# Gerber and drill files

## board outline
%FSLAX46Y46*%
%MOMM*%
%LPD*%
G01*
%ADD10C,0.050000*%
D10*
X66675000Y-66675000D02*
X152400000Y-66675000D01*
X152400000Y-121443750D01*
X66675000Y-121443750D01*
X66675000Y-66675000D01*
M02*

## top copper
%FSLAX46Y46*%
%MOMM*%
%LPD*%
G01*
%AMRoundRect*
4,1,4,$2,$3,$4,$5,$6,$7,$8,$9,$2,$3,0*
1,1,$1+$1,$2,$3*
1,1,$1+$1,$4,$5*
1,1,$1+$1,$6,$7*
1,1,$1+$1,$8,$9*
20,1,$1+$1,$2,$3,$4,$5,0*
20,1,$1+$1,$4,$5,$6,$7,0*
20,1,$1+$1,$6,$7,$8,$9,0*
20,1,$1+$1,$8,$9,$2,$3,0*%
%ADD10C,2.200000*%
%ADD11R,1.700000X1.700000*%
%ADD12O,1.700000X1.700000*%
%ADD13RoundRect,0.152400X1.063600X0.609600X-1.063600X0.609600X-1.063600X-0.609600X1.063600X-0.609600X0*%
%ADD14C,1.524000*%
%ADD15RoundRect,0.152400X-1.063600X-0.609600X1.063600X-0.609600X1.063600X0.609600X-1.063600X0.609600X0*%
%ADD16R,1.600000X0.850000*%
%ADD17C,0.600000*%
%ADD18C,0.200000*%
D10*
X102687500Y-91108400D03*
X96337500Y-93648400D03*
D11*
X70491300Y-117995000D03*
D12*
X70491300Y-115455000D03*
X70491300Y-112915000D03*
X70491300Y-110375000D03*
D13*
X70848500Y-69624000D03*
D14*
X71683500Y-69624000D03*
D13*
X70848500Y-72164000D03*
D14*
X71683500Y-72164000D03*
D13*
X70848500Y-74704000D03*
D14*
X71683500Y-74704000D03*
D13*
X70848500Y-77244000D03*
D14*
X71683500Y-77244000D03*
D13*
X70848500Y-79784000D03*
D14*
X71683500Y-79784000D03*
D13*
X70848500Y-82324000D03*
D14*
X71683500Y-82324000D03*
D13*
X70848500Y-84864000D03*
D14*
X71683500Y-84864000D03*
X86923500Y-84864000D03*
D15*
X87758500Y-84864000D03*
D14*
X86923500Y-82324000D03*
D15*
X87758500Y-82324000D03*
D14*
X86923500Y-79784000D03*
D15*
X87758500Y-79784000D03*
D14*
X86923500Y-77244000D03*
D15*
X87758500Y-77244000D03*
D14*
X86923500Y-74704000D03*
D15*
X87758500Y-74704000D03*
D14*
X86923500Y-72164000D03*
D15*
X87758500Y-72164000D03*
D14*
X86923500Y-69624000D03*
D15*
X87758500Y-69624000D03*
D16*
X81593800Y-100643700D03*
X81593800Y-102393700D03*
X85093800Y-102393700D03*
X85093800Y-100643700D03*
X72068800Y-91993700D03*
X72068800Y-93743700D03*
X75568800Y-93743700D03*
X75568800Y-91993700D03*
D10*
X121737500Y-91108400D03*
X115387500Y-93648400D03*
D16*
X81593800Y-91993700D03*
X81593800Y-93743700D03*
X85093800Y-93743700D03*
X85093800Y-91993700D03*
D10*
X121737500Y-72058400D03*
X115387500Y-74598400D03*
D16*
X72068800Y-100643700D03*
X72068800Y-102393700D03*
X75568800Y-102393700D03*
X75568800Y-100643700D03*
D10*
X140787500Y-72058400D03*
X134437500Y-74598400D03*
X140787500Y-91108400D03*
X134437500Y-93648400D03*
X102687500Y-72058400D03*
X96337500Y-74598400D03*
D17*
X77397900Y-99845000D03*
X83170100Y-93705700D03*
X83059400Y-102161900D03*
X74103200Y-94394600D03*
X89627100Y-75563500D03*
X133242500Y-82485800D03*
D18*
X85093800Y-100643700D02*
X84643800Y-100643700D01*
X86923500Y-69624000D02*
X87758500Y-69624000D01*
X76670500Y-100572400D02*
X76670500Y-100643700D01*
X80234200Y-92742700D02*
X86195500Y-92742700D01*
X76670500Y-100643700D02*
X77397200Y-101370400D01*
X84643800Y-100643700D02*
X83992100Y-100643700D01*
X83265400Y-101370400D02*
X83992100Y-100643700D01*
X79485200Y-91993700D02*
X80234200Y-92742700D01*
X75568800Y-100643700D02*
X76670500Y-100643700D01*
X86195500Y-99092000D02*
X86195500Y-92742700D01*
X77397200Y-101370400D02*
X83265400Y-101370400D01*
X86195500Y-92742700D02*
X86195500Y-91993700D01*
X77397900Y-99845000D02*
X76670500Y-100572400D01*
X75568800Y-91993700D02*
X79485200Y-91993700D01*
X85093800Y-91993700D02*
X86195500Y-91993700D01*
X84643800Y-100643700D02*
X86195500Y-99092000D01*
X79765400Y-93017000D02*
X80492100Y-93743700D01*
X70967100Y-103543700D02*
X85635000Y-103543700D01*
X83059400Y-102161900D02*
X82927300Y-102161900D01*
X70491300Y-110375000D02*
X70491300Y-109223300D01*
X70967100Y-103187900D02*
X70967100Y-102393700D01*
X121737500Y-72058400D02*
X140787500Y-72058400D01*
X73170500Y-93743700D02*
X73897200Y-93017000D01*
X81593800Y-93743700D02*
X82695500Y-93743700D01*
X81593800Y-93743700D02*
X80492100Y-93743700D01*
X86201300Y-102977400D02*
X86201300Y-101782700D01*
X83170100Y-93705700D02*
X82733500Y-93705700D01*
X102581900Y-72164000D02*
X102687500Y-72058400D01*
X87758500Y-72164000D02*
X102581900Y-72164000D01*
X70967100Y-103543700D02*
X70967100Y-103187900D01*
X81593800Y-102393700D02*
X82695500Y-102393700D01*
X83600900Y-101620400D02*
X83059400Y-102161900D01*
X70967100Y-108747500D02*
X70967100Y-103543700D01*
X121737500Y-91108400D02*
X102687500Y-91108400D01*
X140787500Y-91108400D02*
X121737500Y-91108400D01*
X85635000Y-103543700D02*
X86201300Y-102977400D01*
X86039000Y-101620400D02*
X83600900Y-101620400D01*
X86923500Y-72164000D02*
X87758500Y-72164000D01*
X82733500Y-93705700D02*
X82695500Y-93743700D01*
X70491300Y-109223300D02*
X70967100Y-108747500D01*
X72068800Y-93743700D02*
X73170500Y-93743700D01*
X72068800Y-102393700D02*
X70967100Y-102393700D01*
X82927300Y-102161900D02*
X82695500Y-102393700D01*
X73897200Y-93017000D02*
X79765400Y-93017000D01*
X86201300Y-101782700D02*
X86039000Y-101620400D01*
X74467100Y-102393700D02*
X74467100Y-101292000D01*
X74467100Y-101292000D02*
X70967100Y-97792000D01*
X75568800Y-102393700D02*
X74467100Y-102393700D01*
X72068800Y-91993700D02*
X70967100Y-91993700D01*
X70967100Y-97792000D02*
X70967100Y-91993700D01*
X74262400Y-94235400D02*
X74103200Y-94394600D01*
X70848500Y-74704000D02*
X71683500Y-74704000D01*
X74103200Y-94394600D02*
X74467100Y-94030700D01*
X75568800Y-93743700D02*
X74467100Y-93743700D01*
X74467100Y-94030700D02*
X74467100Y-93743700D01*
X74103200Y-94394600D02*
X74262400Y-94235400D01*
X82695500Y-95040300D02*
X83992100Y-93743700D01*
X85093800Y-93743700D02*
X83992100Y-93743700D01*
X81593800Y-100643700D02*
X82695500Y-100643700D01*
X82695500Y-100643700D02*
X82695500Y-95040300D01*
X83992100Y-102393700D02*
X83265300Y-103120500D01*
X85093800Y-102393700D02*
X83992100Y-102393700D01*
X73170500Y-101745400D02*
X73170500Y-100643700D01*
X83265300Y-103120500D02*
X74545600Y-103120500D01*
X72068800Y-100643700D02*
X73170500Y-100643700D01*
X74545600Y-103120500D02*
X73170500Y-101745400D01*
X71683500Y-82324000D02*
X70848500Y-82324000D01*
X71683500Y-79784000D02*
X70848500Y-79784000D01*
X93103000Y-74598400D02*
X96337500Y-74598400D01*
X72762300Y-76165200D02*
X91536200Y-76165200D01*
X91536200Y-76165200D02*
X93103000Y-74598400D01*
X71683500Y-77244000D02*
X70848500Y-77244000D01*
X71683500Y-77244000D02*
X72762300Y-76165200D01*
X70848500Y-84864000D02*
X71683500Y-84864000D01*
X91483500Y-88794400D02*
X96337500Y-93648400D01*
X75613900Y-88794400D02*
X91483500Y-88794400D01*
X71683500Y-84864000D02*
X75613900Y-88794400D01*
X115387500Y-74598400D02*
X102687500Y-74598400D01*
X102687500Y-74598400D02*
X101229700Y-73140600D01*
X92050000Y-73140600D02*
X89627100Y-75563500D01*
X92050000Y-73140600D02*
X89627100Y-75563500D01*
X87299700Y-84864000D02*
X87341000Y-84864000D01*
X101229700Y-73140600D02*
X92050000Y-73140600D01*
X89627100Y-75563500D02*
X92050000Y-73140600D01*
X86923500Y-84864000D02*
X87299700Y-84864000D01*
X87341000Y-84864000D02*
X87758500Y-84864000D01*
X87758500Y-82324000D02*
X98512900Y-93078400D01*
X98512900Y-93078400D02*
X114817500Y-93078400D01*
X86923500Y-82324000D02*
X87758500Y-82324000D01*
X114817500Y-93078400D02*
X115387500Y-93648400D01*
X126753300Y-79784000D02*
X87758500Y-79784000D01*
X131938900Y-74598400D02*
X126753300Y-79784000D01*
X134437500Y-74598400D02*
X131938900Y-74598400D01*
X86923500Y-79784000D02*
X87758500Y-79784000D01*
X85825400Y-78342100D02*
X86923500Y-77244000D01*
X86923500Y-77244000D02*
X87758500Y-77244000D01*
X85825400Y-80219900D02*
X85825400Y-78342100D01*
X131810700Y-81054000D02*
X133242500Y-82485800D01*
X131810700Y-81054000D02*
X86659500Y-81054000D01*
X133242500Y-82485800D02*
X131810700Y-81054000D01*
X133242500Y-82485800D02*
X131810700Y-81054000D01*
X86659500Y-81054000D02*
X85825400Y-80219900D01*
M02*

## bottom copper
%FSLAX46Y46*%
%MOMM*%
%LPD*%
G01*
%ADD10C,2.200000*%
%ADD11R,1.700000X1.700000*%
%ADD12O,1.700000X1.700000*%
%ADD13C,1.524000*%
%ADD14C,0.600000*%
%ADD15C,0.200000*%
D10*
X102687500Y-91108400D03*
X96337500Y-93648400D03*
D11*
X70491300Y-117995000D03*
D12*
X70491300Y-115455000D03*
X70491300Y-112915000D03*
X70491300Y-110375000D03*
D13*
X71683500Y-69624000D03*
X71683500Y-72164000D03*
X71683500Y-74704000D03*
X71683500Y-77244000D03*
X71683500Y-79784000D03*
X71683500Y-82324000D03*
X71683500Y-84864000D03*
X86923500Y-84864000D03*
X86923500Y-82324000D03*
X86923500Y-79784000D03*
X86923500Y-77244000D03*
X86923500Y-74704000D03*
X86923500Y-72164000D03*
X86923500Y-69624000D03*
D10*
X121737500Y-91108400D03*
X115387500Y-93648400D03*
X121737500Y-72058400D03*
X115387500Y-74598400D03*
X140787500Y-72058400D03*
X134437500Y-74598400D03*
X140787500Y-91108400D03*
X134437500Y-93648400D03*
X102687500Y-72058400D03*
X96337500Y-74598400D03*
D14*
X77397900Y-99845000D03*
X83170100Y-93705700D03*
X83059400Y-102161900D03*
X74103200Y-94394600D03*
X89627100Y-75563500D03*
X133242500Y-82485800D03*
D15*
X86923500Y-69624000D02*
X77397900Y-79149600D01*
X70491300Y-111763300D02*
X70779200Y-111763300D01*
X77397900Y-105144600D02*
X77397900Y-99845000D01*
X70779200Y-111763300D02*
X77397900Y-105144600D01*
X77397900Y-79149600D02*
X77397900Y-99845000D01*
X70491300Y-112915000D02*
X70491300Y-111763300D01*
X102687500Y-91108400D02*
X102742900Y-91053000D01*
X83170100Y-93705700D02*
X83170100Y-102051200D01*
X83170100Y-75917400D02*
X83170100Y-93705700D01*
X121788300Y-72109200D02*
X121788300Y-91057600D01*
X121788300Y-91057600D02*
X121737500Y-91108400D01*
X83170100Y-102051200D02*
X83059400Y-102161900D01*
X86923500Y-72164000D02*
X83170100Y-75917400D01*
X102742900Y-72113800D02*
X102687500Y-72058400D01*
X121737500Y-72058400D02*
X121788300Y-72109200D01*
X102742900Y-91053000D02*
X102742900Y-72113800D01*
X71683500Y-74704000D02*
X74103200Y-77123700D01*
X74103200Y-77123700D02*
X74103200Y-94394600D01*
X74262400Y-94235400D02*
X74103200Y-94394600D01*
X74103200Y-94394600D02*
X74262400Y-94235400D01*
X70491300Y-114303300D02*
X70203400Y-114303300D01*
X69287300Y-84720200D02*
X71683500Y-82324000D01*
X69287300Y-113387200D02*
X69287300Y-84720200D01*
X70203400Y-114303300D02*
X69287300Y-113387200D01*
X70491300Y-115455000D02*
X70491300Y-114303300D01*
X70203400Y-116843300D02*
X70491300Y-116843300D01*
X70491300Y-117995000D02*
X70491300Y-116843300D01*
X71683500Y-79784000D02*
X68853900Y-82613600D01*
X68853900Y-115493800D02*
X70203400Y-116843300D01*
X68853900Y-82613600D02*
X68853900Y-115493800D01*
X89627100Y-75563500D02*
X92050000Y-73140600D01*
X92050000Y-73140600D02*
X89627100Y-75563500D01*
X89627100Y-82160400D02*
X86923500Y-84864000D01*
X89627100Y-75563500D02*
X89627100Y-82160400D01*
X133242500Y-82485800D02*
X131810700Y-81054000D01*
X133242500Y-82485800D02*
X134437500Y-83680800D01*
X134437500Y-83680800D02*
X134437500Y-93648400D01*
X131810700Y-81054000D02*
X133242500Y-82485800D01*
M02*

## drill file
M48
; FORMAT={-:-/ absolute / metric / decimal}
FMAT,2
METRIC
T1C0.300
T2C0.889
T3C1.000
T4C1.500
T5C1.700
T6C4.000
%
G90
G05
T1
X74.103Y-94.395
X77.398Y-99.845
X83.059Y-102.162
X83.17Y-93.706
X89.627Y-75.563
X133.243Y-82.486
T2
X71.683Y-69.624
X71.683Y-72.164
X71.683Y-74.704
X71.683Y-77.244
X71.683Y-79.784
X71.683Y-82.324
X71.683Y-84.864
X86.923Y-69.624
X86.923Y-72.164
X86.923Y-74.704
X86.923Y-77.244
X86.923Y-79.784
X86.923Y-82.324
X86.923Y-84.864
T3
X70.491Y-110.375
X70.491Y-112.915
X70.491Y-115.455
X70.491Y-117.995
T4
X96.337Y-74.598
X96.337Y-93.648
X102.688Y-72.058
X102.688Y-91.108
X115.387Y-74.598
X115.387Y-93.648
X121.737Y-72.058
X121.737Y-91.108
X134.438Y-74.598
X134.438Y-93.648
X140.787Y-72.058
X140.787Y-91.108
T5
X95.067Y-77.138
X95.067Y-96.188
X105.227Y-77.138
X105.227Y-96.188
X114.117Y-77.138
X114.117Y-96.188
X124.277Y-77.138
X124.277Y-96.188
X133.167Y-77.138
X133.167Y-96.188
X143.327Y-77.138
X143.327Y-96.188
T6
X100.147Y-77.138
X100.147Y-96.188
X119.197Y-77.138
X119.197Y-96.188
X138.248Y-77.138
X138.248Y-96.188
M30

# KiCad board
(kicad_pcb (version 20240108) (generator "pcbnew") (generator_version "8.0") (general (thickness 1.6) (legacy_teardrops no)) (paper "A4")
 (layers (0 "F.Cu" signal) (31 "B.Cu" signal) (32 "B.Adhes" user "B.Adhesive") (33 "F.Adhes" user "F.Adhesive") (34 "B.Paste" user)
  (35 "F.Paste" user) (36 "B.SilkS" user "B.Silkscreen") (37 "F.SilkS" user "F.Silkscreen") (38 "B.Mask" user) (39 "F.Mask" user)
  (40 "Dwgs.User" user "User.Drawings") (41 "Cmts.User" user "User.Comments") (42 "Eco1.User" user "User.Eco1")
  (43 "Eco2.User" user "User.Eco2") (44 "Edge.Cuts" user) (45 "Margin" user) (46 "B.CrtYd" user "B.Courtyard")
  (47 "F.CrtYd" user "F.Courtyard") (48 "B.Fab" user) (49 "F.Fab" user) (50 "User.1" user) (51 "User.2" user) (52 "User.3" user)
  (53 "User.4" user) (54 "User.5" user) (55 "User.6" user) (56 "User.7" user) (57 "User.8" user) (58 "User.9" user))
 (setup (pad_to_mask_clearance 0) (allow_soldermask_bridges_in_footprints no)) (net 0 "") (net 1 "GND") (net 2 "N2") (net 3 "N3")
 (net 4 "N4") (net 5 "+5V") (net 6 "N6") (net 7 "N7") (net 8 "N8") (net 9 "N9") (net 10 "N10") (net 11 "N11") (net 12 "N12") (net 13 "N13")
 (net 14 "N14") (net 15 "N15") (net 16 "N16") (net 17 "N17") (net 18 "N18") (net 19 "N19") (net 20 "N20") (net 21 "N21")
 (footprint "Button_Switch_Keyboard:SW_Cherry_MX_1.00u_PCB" (layer "F.Cu") (at 102.6875 91.1084)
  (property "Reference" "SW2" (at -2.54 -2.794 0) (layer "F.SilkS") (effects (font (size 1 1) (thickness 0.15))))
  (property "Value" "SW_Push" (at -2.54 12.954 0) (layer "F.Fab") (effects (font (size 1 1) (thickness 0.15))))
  (pad "" np_thru_hole circle (at -7.62 5.08) (size 1.7 1.7) (drill 1.7) (layers "*.Cu" "*.Mask"))
  (pad "" np_thru_hole circle (at -2.54 5.08) (size 4 4) (drill 4) (layers "*.Cu" "*.Mask"))
  (pad "" np_thru_hole circle (at 2.54 5.08) (size 1.7 1.7) (drill 1.7) (layers "*.Cu" "*.Mask"))
  (pad "1" thru_hole circle (at 0 0) (size 2.2 2.2) (drill 1.5) (layers "*.Cu" "*.Mask") (remove_unused_layers no) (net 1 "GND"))
  (pad "2" thru_hole circle (at -6.35 2.54) (size 2.2 2.2) (drill 1.5) (layers "*.Cu" "*.Mask") (remove_unused_layers no) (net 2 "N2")))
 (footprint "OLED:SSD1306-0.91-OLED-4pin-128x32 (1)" (layer "F.Cu") (at 106.9913 120.185 180)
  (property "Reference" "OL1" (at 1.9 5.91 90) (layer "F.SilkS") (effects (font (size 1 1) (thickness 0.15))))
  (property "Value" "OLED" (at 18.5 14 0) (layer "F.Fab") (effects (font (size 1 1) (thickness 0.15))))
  (pad "1" thru_hole rect (at 36.5 2.19 180) (size 1.7 1.7) (drill 1) (layers "*.Cu" "*.Mask") (remove_unused_layers no) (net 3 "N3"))
  (pad "2" thru_hole oval (at 36.5 4.73 180) (size 1.7 1.7) (drill 1) (layers "*.Cu" "*.Mask") (remove_unused_layers no) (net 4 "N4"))
  (pad "3" thru_hole oval (at 36.5 7.27 180) (size 1.7 1.7) (drill 1) (layers "*.Cu" "*.Mask") (remove_unused_layers no) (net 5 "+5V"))
  (pad "4" thru_hole oval (at 36.5 9.81 180) (size 1.7 1.7) (drill 1) (layers "*.Cu" "*.Mask") (remove_unused_layers no) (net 1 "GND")))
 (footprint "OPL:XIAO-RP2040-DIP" (layer "F.Cu") (at 79.3035 77.244)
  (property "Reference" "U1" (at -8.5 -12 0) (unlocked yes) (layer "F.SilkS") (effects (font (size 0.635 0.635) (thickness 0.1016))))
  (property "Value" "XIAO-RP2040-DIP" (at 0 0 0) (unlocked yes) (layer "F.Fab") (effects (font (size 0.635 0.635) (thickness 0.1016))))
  (pad "1" smd roundrect (at -8.455 -7.62 180) (size 2.432 1.524) (layers "F.Cu" "F.Mask") (roundrect_rratio 0.1) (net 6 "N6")
   (thermal_bridge_angle 45))
  (pad "1" thru_hole circle (at -7.62 -7.62 180) (size 1.524 1.524) (drill 0.889) (layers "*.Cu" "*.Mask") (remove_unused_layers no)
   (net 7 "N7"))
  (pad "2" smd roundrect (at -8.455 -5.08 180) (size 2.432 1.524) (layers "F.Cu" "F.Mask") (roundrect_rratio 0.1) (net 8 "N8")
   (thermal_bridge_angle 45))
  (pad "2" thru_hole circle (at -7.62 -5.08 180) (size 1.524 1.524) (drill 0.889) (layers "*.Cu" "*.Mask") (remove_unused_layers no)
   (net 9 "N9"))
  (pad "3" smd roundrect (at -8.455 -2.54 180) (size 2.432 1.524) (layers "F.Cu" "F.Mask") (roundrect_rratio 0.1) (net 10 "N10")
   (thermal_bridge_angle 45))
  (pad "3" thru_hole circle (at -7.62 -2.54 180) (size 1.524 1.524) (drill 0.889) (layers "*.Cu" "*.Mask") (remove_unused_layers no)
   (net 10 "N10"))
  (pad "4" smd roundrect (at -8.455 0 180) (size 2.432 1.524) (layers "F.Cu" "F.Mask") (roundrect_rratio 0.1) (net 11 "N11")
   (thermal_bridge_angle 45))
  (pad "4" thru_hole circle (at -7.62 0 180) (size 1.524 1.524) (drill 0.889) (layers "*.Cu" "*.Mask") (remove_unused_layers no)
   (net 11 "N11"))
  (pad "5" smd roundrect (at -8.455 2.54 180) (size 2.432 1.524) (layers "F.Cu" "F.Mask") (roundrect_rratio 0.1) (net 3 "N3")
   (thermal_bridge_angle 45))
  (pad "5" thru_hole circle (at -7.62 2.54 180) (size 1.524 1.524) (drill 0.889) (layers "*.Cu" "*.Mask") (remove_unused_layers no)
   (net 3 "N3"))
  (pad "6" smd roundrect (at -8.455 5.08 180) (size 2.432 1.524) (layers "F.Cu" "F.Mask") (roundrect_rratio 0.1) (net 4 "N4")
   (thermal_bridge_angle 45))
  (pad "6" thru_hole circle (at -7.62 5.08 180) (size 1.524 1.524) (drill 0.889) (layers "*.Cu" "*.Mask") (remove_unused_layers no)
   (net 4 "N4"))
  (pad "7" smd roundrect (at -8.455 7.62 180) (size 2.432 1.524) (layers "F.Cu" "F.Mask") (roundrect_rratio 0.1) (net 2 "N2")
   (thermal_bridge_angle 45))
  (pad "7" thru_hole circle (at -7.62 7.62 180) (size 1.524 1.524) (drill 0.889) (layers "*.Cu" "*.Mask") (remove_unused_layers no)
   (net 2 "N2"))
  (pad "8" thru_hole circle (at 7.62 7.62) (size 1.524 1.524) (drill 0.889) (layers "*.Cu" "*.Mask") (remove_unused_layers no)
   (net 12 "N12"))
  (pad "8" smd roundrect (at 8.455 7.62) (size 2.432 1.524) (layers "F.Cu" "F.Mask") (roundrect_rratio 0.1) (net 12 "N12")
   (thermal_bridge_angle 45))
  (pad "9" thru_hole circle (at 7.62 5.08) (size 1.524 1.524) (drill 0.889) (layers "*.Cu" "*.Mask") (remove_unused_layers no)
   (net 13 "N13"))
  (pad "9" smd roundrect (at 8.455 5.08) (size 2.432 1.524) (layers "F.Cu" "F.Mask") (roundrect_rratio 0.1) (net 13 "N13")
   (thermal_bridge_angle 45))
  (pad "10" thru_hole circle (at 7.62 2.54) (size 1.524 1.524) (drill 0.889) (layers "*.Cu" "*.Mask") (remove_unused_layers no)
   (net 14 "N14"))
  (pad "10" smd roundrect (at 8.455 2.54) (size 2.432 1.524) (layers "F.Cu" "F.Mask") (roundrect_rratio 0.1) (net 14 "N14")
   (thermal_bridge_angle 45))
  (pad "11" thru_hole circle (at 7.62 0) (size 1.524 1.524) (drill 0.889) (layers "*.Cu" "*.Mask") (remove_unused_layers no) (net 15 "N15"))
  (pad "11" smd roundrect (at 8.455 0) (size 2.432 1.524) (layers "F.Cu" "F.Mask") (roundrect_rratio 0.1) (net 15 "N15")
   (thermal_bridge_angle 45))
  (pad "12" thru_hole circle (at 7.62 -2.54) (size 1.524 1.524) (drill 0.889) (layers "*.Cu" "*.Mask") (remove_unused_layers no)
   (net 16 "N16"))
  (pad "12" smd roundrect (at 8.455 -2.54) (size 2.432 1.524) (layers "F.Cu" "F.Mask") (roundrect_rratio 0.1) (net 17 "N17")
   (thermal_bridge_angle 45))
  (pad "13" thru_hole circle (at 7.62 -5.08) (size 1.524 1.524) (drill 0.889) (layers "*.Cu" "*.Mask") (remove_unused_layers no)
   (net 1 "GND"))
  (pad "13" smd roundrect (at 8.455 -5.08) (size 2.432 1.524) (layers "F.Cu" "F.Mask") (roundrect_rratio 0.1) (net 1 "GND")
   (thermal_bridge_angle 45))
  (pad "14" thru_hole circle (at 7.62 -7.62) (size 1.524 1.524) (drill 0.889) (layers "*.Cu" "*.Mask") (remove_unused_layers no)
   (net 5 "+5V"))
  (pad "14" smd roundrect (at 8.455 -7.62) (size 2.432 1.524) (layers "F.Cu" "F.Mask") (roundrect_rratio 0.1) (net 5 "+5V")
   (thermal_bridge_angle 45)))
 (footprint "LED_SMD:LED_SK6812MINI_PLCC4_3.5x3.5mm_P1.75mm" (layer "F.Cu") (at 83.3438 101.5187)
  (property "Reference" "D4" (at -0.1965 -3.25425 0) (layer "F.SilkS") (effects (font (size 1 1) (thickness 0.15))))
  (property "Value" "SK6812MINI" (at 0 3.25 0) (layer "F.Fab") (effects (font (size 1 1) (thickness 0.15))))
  (pad "1" smd rect (at -1.75 -0.875) (size 1.6 0.85) (layers "F.Cu" "F.Paste" "F.Mask") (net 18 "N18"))
  (pad "2" smd rect (at -1.75 0.875) (size 1.6 0.85) (layers "F.Cu" "F.Paste" "F.Mask") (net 1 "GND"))
  (pad "3" smd rect (at 1.75 0.875) (size 1.6 0.85) (layers "F.Cu" "F.Paste" "F.Mask") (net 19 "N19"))
  (pad "4" smd rect (at 1.75 -0.875) (size 1.6 0.85) (layers "F.Cu" "F.Paste" "F.Mask") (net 5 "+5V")))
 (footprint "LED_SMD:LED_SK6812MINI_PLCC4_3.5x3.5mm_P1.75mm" (layer "F.Cu") (at 73.8188 92.8687)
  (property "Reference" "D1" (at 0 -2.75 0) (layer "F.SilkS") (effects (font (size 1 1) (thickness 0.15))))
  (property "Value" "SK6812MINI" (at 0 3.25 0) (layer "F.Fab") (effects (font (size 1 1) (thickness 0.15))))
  (pad "1" smd rect (at -1.75 -0.875) (size 1.6 0.85) (layers "F.Cu" "F.Paste" "F.Mask") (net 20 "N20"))
  (pad "2" smd rect (at -1.75 0.875) (size 1.6 0.85) (layers "F.Cu" "F.Paste" "F.Mask") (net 1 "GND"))
  (pad "3" smd rect (at 1.75 0.875) (size 1.6 0.85) (layers "F.Cu" "F.Paste" "F.Mask") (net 10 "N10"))
  (pad "4" smd rect (at 1.75 -0.875) (size 1.6 0.85) (layers "F.Cu" "F.Paste" "F.Mask") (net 5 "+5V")))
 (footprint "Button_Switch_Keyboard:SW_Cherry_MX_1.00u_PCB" (layer "F.Cu") (at 121.7375 91.1084)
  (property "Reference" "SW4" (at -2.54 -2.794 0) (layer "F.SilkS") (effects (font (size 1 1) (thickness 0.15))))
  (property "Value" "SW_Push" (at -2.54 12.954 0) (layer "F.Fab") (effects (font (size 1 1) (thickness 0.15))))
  (pad "" np_thru_hole circle (at -7.62 5.08) (size 1.7 1.7) (drill 1.7) (layers "*.Cu" "*.Mask"))
  (pad "" np_thru_hole circle (at -2.54 5.08) (size 4 4) (drill 4) (layers "*.Cu" "*.Mask"))
  (pad "" np_thru_hole circle (at 2.54 5.08) (size 1.7 1.7) (drill 1.7) (layers "*.Cu" "*.Mask"))
  (pad "1" thru_hole circle (at 0 0) (size 2.2 2.2) (drill 1.5) (layers "*.Cu" "*.Mask") (remove_unused_layers no) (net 1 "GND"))
  (pad "2" thru_hole circle (at -6.35 2.54) (size 2.2 2.2) (drill 1.5) (layers "*.Cu" "*.Mask") (remove_unused_layers no) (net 13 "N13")))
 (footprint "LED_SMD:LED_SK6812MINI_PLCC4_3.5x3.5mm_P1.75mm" (layer "F.Cu") (at 83.3438 92.8687)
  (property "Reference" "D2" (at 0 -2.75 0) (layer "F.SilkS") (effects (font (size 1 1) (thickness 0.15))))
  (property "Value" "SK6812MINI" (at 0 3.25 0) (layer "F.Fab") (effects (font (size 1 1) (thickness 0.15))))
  (pad "1" smd rect (at -1.75 -0.875) (size 1.6 0.85) (layers "F.Cu" "F.Paste" "F.Mask") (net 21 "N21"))
  (pad "2" smd rect (at -1.75 0.875) (size 1.6 0.85) (layers "F.Cu" "F.Paste" "F.Mask") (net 1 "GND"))
  (pad "3" smd rect (at 1.75 0.875) (size 1.6 0.85) (layers "F.Cu" "F.Paste" "F.Mask") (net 18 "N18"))
  (pad "4" smd rect (at 1.75 -0.875) (size 1.6 0.85) (layers "F.Cu" "F.Paste" "F.Mask") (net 5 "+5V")))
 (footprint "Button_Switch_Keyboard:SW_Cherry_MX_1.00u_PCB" (layer "F.Cu") (at 121.7375 72.0584)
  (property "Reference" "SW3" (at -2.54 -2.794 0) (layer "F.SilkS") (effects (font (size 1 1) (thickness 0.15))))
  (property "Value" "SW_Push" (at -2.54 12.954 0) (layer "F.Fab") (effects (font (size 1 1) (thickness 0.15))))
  (pad "" np_thru_hole circle (at -7.62 5.08) (size 1.7 1.7) (drill 1.7) (layers "*.Cu" "*.Mask"))
  (pad "" np_thru_hole circle (at -2.54 5.08) (size 4 4) (drill 4) (layers "*.Cu" "*.Mask"))
  (pad "" np_thru_hole circle (at 2.54 5.08) (size 1.7 1.7) (drill 1.7) (layers "*.Cu" "*.Mask"))
  (pad "1" thru_hole circle (at 0 0) (size 2.2 2.2) (drill 1.5) (layers "*.Cu" "*.Mask") (remove_unused_layers no) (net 1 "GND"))
  (pad "2" thru_hole circle (at -6.35 2.54) (size 2.2 2.2) (drill 1.5) (layers "*.Cu" "*.Mask") (remove_unused_layers no) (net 12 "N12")))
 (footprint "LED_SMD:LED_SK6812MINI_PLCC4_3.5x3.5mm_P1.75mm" (layer "F.Cu") (at 73.8188 101.5187)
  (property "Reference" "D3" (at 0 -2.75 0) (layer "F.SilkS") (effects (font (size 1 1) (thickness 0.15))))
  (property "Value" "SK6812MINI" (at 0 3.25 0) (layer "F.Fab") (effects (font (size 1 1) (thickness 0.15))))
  (pad "1" smd rect (at -1.75 -0.875) (size 1.6 0.85) (layers "F.Cu" "F.Paste" "F.Mask") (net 19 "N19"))
  (pad "2" smd rect (at -1.75 0.875) (size 1.6 0.85) (layers "F.Cu" "F.Paste" "F.Mask") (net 1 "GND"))
  (pad "3" smd rect (at 1.75 0.875) (size 1.6 0.85) (layers "F.Cu" "F.Paste" "F.Mask") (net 20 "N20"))
  (pad "4" smd rect (at 1.75 -0.875) (size 1.6 0.85) (layers "F.Cu" "F.Paste" "F.Mask") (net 5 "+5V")))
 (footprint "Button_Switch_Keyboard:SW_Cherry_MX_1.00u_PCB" (layer "F.Cu") (at 140.7875 72.0584)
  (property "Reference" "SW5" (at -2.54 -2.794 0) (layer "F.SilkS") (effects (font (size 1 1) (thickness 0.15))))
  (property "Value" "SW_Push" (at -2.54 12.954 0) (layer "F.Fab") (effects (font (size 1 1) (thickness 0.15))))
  (pad "" np_thru_hole circle (at -7.62 5.08) (size 1.7 1.7) (drill 1.7) (layers "*.Cu" "*.Mask"))
  (pad "" np_thru_hole circle (at -2.54 5.08) (size 4 4) (drill 4) (layers "*.Cu" "*.Mask"))
  (pad "" np_thru_hole circle (at 2.54 5.08) (size 1.7 1.7) (drill 1.7) (layers "*.Cu" "*.Mask"))
  (pad "1" thru_hole circle (at 0 0) (size 2.2 2.2) (drill 1.5) (layers "*.Cu" "*.Mask") (remove_unused_layers no) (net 1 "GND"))
  (pad "2" thru_hole circle (at -6.35 2.54) (size 2.2 2.2) (drill 1.5) (layers "*.Cu" "*.Mask") (remove_unused_layers no) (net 14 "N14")))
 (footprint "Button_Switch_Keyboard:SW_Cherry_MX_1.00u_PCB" (layer "F.Cu") (at 140.7875 91.1084)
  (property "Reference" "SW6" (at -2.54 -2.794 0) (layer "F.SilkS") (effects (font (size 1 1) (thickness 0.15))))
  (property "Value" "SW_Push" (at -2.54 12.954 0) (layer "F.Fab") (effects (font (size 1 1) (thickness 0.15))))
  (pad "" np_thru_hole circle (at -7.62 5.08) (size 1.7 1.7) (drill 1.7) (layers "*.Cu" "*.Mask"))
  (pad "" np_thru_hole circle (at -2.54 5.08) (size 4 4) (drill 4) (layers "*.Cu" "*.Mask"))
  (pad "" np_thru_hole circle (at 2.54 5.08) (size 1.7 1.7) (drill 1.7) (layers "*.Cu" "*.Mask"))
  (pad "1" thru_hole circle (at 0 0) (size 2.2 2.2) (drill 1.5) (layers "*.Cu" "*.Mask") (remove_unused_layers no) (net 1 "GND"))
  (pad "2" thru_hole circle (at -6.35 2.54) (size 2.2 2.2) (drill 1.5) (layers "*.Cu" "*.Mask") (remove_unused_layers no) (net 15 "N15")))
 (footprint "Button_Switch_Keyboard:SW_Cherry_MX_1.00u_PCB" (layer "F.Cu") (at 102.6875 72.0584)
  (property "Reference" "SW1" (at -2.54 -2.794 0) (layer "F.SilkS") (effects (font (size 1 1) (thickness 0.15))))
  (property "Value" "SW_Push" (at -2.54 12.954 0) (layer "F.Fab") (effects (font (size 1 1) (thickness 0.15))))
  (pad "" np_thru_hole circle (at -7.62 5.08) (size 1.7 1.7) (drill 1.7) (layers "*.Cu" "*.Mask"))
  (pad "" np_thru_hole circle (at -2.54 5.08) (size 4 4) (drill 4) (layers "*.Cu" "*.Mask"))
  (pad "" np_thru_hole circle (at 2.54 5.08) (size 1.7 1.7) (drill 1.7) (layers "*.Cu" "*.Mask"))
  (pad "1" thru_hole circle (at 0 0) (size 2.2 2.2) (drill 1.5) (layers "*.Cu" "*.Mask") (remove_unused_layers no) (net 1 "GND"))
  (pad "2" thru_hole circle (at -6.35 2.54) (size 2.2 2.2) (drill 1.5) (layers "*.Cu" "*.Mask") (remove_unused_layers no) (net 11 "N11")))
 (gr_rect (start 66.675 66.675) (end 152.4 121.44375) (stroke (width 0.05) (type default)) (fill none) (layer "Edge.Cuts"))
 (segment (start 85.0938 100.6437) (end 84.6438 100.6437) (width 0.2) (layer "F.Cu") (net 5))
 (segment (start 86.9235 69.624) (end 87.7585 69.624) (width 0.2) (layer "F.Cu") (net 5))
 (segment (start 76.6705 100.5724) (end 76.6705 100.6437) (width 0.2) (layer "F.Cu") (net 5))
 (segment (start 80.2342 92.7427) (end 86.1955 92.7427) (width 0.2) (layer "F.Cu") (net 5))
 (segment (start 76.6705 100.6437) (end 77.3972 101.3704) (width 0.2) (layer "F.Cu") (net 5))
 (segment (start 84.6438 100.6437) (end 83.9921 100.6437) (width 0.2) (layer "F.Cu") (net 5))
 (segment (start 83.2654 101.3704) (end 83.9921 100.6437) (width 0.2) (layer "F.Cu") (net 5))
 (segment (start 79.4852 91.9937) (end 80.2342 92.7427) (width 0.2) (layer "F.Cu") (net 5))
 (segment (start 75.5688 100.6437) (end 76.6705 100.6437) (width 0.2) (layer "F.Cu") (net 5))
 (segment (start 86.1955 99.092) (end 86.1955 92.7427) (width 0.2) (layer "F.Cu") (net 5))
 (segment (start 77.3972 101.3704) (end 83.2654 101.3704) (width 0.2) (layer "F.Cu") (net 5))
 (segment (start 86.1955 92.7427) (end 86.1955 91.9937) (width 0.2) (layer "F.Cu") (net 5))
 (segment (start 77.3979 99.845) (end 76.6705 100.5724) (width 0.2) (layer "F.Cu") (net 5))
 (segment (start 75.5688 91.9937) (end 79.4852 91.9937) (width 0.2) (layer "F.Cu") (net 5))
 (segment (start 85.0938 91.9937) (end 86.1955 91.9937) (width 0.2) (layer "F.Cu") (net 5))
 (segment (start 84.6438 100.6437) (end 86.1955 99.092) (width 0.2) (layer "F.Cu") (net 5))
 (via (at 77.3979 99.845) (size 0.6) (drill 0.3) (layers "F.Cu" "B.Cu") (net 5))
 (segment (start 86.9235 69.624) (end 77.3979 79.1496) (width 0.2) (layer "B.Cu") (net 5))
 (segment (start 70.4913 111.7633) (end 70.7792 111.7633) (width 0.2) (layer "B.Cu") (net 5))
 (segment (start 77.3979 105.1446) (end 77.3979 99.845) (width 0.2) (layer "B.Cu") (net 5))
 (segment (start 70.7792 111.7633) (end 77.3979 105.1446) (width 0.2) (layer "B.Cu") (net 5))
 (segment (start 77.3979 79.1496) (end 77.3979 99.845) (width 0.2) (layer "B.Cu") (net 5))
 (segment (start 70.4913 112.915) (end 70.4913 111.7633) (width 0.2) (layer "B.Cu") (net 5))
 (segment (start 79.7654 93.017) (end 80.4921 93.7437) (width 0.2) (layer "F.Cu") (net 1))
 (segment (start 70.9671 103.5437) (end 85.635 103.5437) (width 0.2) (layer "F.Cu") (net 1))
 (segment (start 83.0594 102.1619) (end 82.9273 102.1619) (width 0.2) (layer "F.Cu") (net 1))
 (segment (start 70.4913 110.375) (end 70.4913 109.2233) (width 0.2) (layer "F.Cu") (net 1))
 (segment (start 70.9671 103.1879) (end 70.9671 102.3937) (width 0.2) (layer "F.Cu") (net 1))
 (segment (start 121.7375 72.0584) (end 140.7875 72.0584) (width 0.2) (layer "F.Cu") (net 1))
 (segment (start 73.1705 93.7437) (end 73.8972 93.017) (width 0.2) (layer "F.Cu") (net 1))
 (segment (start 81.5938 93.7437) (end 82.6955 93.7437) (width 0.2) (layer "F.Cu") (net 1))
 (segment (start 81.5938 93.7437) (end 80.4921 93.7437) (width 0.2) (layer "F.Cu") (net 1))
 (segment (start 86.2013 102.9774) (end 86.2013 101.7827) (width 0.2) (layer "F.Cu") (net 1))
 (segment (start 83.1701 93.7057) (end 82.7335 93.7057) (width 0.2) (layer "F.Cu") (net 1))
 (segment (start 102.5819 72.164) (end 102.6875 72.0584) (width 0.2) (layer "F.Cu") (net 1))
 (segment (start 87.7585 72.164) (end 102.5819 72.164) (width 0.2) (layer "F.Cu") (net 1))
 (segment (start 70.9671 103.5437) (end 70.9671 103.1879) (width 0.2) (layer "F.Cu") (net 1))
 (segment (start 81.5938 102.3937) (end 82.6955 102.3937) (width 0.2) (layer "F.Cu") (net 1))
 (segment (start 83.6009 101.6204) (end 83.0594 102.1619) (width 0.2) (layer "F.Cu") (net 1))
 (segment (start 70.9671 108.7475) (end 70.9671 103.5437) (width 0.2) (layer "F.Cu") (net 1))
 (segment (start 121.7375 91.1084) (end 102.6875 91.1084) (width 0.2) (layer "F.Cu") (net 1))
 (segment (start 140.7875 91.1084) (end 121.7375 91.1084) (width 0.2) (layer "F.Cu") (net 1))
 (segment (start 85.635 103.5437) (end 86.2013 102.9774) (width 0.2) (layer "F.Cu") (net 1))
 (segment (start 86.039 101.6204) (end 83.6009 101.6204) (width 0.2) (layer "F.Cu") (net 1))
 (segment (start 86.9235 72.164) (end 87.7585 72.164) (width 0.2) (layer "F.Cu") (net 1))
 (segment (start 82.7335 93.7057) (end 82.6955 93.7437) (width 0.2) (layer "F.Cu") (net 1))
 (segment (start 70.4913 109.2233) (end 70.9671 108.7475) (width 0.2) (layer "F.Cu") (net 1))
 (segment (start 72.0688 93.7437) (end 73.1705 93.7437) (width 0.2) (layer "F.Cu") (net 1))
 (segment (start 72.0688 102.3937) (end 70.9671 102.3937) (width 0.2) (layer "F.Cu") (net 1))
 (segment (start 82.9273 102.1619) (end 82.6955 102.3937) (width 0.2) (layer "F.Cu") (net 1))
 (segment (start 73.8972 93.017) (end 79.7654 93.017) (width 0.2) (layer "F.Cu") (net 1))
 (segment (start 86.2013 101.7827) (end 86.039 101.6204) (width 0.2) (layer "F.Cu") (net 1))
 (via (at 83.1701 93.7057) (size 0.6) (drill 0.3) (layers "F.Cu" "B.Cu") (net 1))
 (via (at 83.0594 102.1619) (size 0.6) (drill 0.3) (layers "F.Cu" "B.Cu") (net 1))
 (segment (start 102.6875 91.1084) (end 102.7429 91.053) (width 0.2) (layer "B.Cu") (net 1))
 (segment (start 83.1701 93.7057) (end 83.1701 102.0512) (width 0.2) (layer "B.Cu") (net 1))
 (segment (start 83.1701 75.9174) (end 83.1701 93.7057) (width 0.2) (layer "B.Cu") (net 1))
 (segment (start 121.7883 72.1092) (end 121.7883 91.0576) (width 0.2) (layer "B.Cu") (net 1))
 (segment (start 121.7883 91.0576) (end 121.7375 91.1084) (width 0.2) (layer "B.Cu") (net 1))
 (segment (start 83.1701 102.0512) (end 83.0594 102.1619) (width 0.2) (layer "B.Cu") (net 1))
 (segment (start 86.9235 72.164) (end 83.1701 75.9174) (width 0.2) (layer "B.Cu") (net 1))
 (segment (start 102.7429 72.1138) (end 102.6875 72.0584) (width 0.2) (layer "B.Cu") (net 1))
 (segment (start 121.7375 72.0584) (end 121.7883 72.1092) (width 0.2) (layer "B.Cu") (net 1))
 (segment (start 102.7429 91.053) (end 102.7429 72.1138) (width 0.2) (layer "B.Cu") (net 1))
 (segment (start 74.4671 102.3937) (end 74.4671 101.292) (width 0.2) (layer "F.Cu") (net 20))
 (segment (start 74.4671 101.292) (end 70.9671 97.792) (width 0.2) (layer "F.Cu") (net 20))
 (segment (start 75.5688 102.3937) (end 74.4671 102.3937) (width 0.2) (layer "F.Cu") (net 20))
 (segment (start 72.0688 91.9937) (end 70.9671 91.9937) (width 0.2) (layer "F.Cu") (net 20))
 (segment (start 70.9671 97.792) (end 70.9671 91.9937) (width 0.2) (layer "F.Cu") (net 20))
 (segment (start 74.2624 94.2354) (end 74.1032 94.3946) (width 0.2) (layer "F.Cu") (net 10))
 (segment (start 70.8485 74.704) (end 71.6835 74.704) (width 0.2) (layer "F.Cu") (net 10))
 (segment (start 74.1032 94.3946) (end 74.4671 94.0307) (width 0.2) (layer "F.Cu") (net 10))
 (segment (start 75.5688 93.7437) (end 74.4671 93.7437) (width 0.2) (layer "F.Cu") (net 10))
 (segment (start 74.4671 94.0307) (end 74.4671 93.7437) (width 0.2) (layer "F.Cu") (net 10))
 (segment (start 74.1032 94.3946) (end 74.2624 94.2354) (width 0.2) (layer "F.Cu") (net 10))
 (via (at 74.1032 94.3946) (size 0.6) (drill 0.3) (layers "F.Cu" "B.Cu") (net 10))
 (segment (start 71.6835 74.704) (end 74.1032 77.1237) (width 0.2) (layer "B.Cu") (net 10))
 (segment (start 74.1032 77.1237) (end 74.1032 94.3946) (width 0.2) (layer "B.Cu") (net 10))
 (segment (start 74.2624 94.2354) (end 74.1032 94.3946) (width 0.2) (layer "B.Cu") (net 10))
 (segment (start 74.1032 94.3946) (end 74.2624 94.2354) (width 0.2) (layer "B.Cu") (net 10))
 (segment (start 82.6955 95.0403) (end 83.9921 93.7437) (width 0.2) (layer "F.Cu") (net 18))
 (segment (start 85.0938 93.7437) (end 83.9921 93.7437) (width 0.2) (layer "F.Cu") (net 18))
 (segment (start 81.5938 100.6437) (end 82.6955 100.6437) (width 0.2) (layer "F.Cu") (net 18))
 (segment (start 82.6955 100.6437) (end 82.6955 95.0403) (width 0.2) (layer "F.Cu") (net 18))
 (segment (start 83.9921 102.3937) (end 83.2653 103.1205) (width 0.2) (layer "F.Cu") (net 19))
 (segment (start 85.0938 102.3937) (end 83.9921 102.3937) (width 0.2) (layer "F.Cu") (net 19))
 (segment (start 73.1705 101.7454) (end 73.1705 100.6437) (width 0.2) (layer "F.Cu") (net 19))
 (segment (start 83.2653 103.1205) (end 74.5456 103.1205) (width 0.2) (layer "F.Cu") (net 19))
 (segment (start 72.0688 100.6437) (end 73.1705 100.6437) (width 0.2) (layer "F.Cu") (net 19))
 (segment (start 74.5456 103.1205) (end 73.1705 101.7454) (width 0.2) (layer "F.Cu") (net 19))
 (segment (start 71.6835 82.324) (end 70.8485 82.324) (width 0.2) (layer "F.Cu") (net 4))
 (segment (start 70.4913 114.3033) (end 70.2034 114.3033) (width 0.2) (layer "B.Cu") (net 4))
 (segment (start 69.2873 84.7202) (end 71.6835 82.324) (width 0.2) (layer "B.Cu") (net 4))
 (segment (start 69.2873 113.3872) (end 69.2873 84.7202) (width 0.2) (layer "B.Cu") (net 4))
 (segment (start 70.2034 114.3033) (end 69.2873 113.3872) (width 0.2) (layer "B.Cu") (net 4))
 (segment (start 70.4913 115.455) (end 70.4913 114.3033) (width 0.2) (layer "B.Cu") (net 4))
 (segment (start 71.6835 79.784) (end 70.8485 79.784) (width 0.2) (layer "F.Cu") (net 3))
 (segment (start 70.2034 116.8433) (end 70.4913 116.8433) (width 0.2) (layer "B.Cu") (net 3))
 (segment (start 70.4913 117.995) (end 70.4913 116.8433) (width 0.2) (layer "B.Cu") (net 3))
 (segment (start 71.6835 79.784) (end 68.8539 82.6136) (width 0.2) (layer "B.Cu") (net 3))
 (segment (start 68.8539 115.4938) (end 70.2034 116.8433) (width 0.2) (layer "B.Cu") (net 3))
 (segment (start 68.8539 82.6136) (end 68.8539 115.4938) (width 0.2) (layer "B.Cu") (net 3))
 (segment (start 93.103 74.5984) (end 96.3375 74.5984) (width 0.2) (layer "F.Cu") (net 11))
 (segment (start 72.7623 76.1652) (end 91.5362 76.1652) (width 0.2) (layer "F.Cu") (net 11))
 (segment (start 91.5362 76.1652) (end 93.103 74.5984) (width 0.2) (layer "F.Cu") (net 11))
 (segment (start 71.6835 77.244) (end 70.8485 77.244) (width 0.2) (layer "F.Cu") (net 11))
 (segment (start 71.6835 77.244) (end 72.7623 76.1652) (width 0.2) (layer "F.Cu") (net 11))
 (segment (start 70.8485 84.864) (end 71.6835 84.864) (width 0.2) (layer "F.Cu") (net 2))
 (segment (start 91.4835 88.7944) (end 96.3375 93.6484) (width 0.2) (layer "F.Cu") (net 2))
 (segment (start 75.6139 88.7944) (end 91.4835 88.7944) (width 0.2) (layer "F.Cu") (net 2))
 (segment (start 71.6835 84.864) (end 75.6139 88.7944) (width 0.2) (layer "F.Cu") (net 2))
 (segment (start 115.3875 74.5984) (end 102.6875 74.5984) (width 0.2) (layer "F.Cu") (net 12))
 (segment (start 102.6875 74.5984) (end 101.2297 73.1406) (width 0.2) (layer "F.Cu") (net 12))
 (segment (start 92.05 73.1406) (end 89.6271 75.5635) (width 0.2) (layer "F.Cu") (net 12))
 (segment (start 92.05 73.1406) (end 89.6271 75.5635) (width 0.2) (layer "F.Cu") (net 12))
 (segment (start 87.2997 84.864) (end 87.341 84.864) (width 0.2) (layer "F.Cu") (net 12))
 (segment (start 101.2297 73.1406) (end 92.05 73.1406) (width 0.2) (layer "F.Cu") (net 12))
 (segment (start 89.6271 75.5635) (end 92.05 73.1406) (width 0.2) (layer "F.Cu") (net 12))
 (segment (start 86.9235 84.864) (end 87.2997 84.864) (width 0.2) (layer "F.Cu") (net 12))
 (segment (start 87.341 84.864) (end 87.7585 84.864) (width 0.2) (layer "F.Cu") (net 12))
 (via (at 89.6271 75.5635) (size 0.6) (drill 0.3) (layers "F.Cu" "B.Cu") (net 12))
 (segment (start 89.6271 75.5635) (end 92.05 73.1406) (width 0.2) (layer "B.Cu") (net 12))
 (segment (start 92.05 73.1406) (end 89.6271 75.5635) (width 0.2) (layer "B.Cu") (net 12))
 (segment (start 89.6271 82.1604) (end 86.9235 84.864) (width 0.2) (layer "B.Cu") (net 12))
 (segment (start 89.6271 75.5635) (end 89.6271 82.1604) (width 0.2) (layer "B.Cu") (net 12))
 (segment (start 87.7585 82.324) (end 98.5129 93.0784) (width 0.2) (layer "F.Cu") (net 13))
 (segment (start 98.5129 93.0784) (end 114.8175 93.0784) (width 0.2) (layer "F.Cu") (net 13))
 (segment (start 86.9235 82.324) (end 87.7585 82.324) (width 0.2) (layer "F.Cu") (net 13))
 (segment (start 114.8175 93.0784) (end 115.3875 93.6484) (width 0.2) (layer "F.Cu") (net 13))
 (segment (start 126.7533 79.784) (end 87.7585 79.784) (width 0.2) (layer "F.Cu") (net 14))
 (segment (start 131.9389 74.5984) (end 126.7533 79.784) (width 0.2) (layer "F.Cu") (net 14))
 (segment (start 134.4375 74.5984) (end 131.9389 74.5984) (width 0.2) (layer "F.Cu") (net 14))
 (segment (start 86.9235 79.784) (end 87.7585 79.784) (width 0.2) (layer "F.Cu") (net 14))
 (segment (start 85.8254 78.3421) (end 86.9235 77.244) (width 0.2) (layer "F.Cu") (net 15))
 (segment (start 86.9235 77.244) (end 87.7585 77.244) (width 0.2) (layer "F.Cu") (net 15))
 (segment (start 85.8254 80.2199) (end 85.8254 78.3421) (width 0.2) (layer "F.Cu") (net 15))
 (segment (start 131.8107 81.054) (end 133.2425 82.4858) (width 0.2) (layer "F.Cu") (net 15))
 (segment (start 131.8107 81.054) (end 86.6595 81.054) (width 0.2) (layer "F.Cu") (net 15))
 (segment (start 133.2425 82.4858) (end 131.8107 81.054) (width 0.2) (layer "F.Cu") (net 15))
 (segment (start 133.2425 82.4858) (end 131.8107 81.054) (width 0.2) (layer "F.Cu") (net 15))
 (segment (start 86.6595 81.054) (end 85.8254 80.2199) (width 0.2) (layer "F.Cu") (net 15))
 (via (at 133.2425 82.4858) (size 0.6) (drill 0.3) (layers "F.Cu" "B.Cu") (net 15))
 (segment (start 133.2425 82.4858) (end 131.8107 81.054) (width 0.2) (layer "B.Cu") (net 15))
 (segment (start 133.2425 82.4858) (end 134.4375 83.6808) (width 0.2) (layer "B.Cu") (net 15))
 (segment (start 134.4375 83.6808) (end 134.4375 93.6484) (width 0.2) (layer "B.Cu") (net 15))
 (segment (start 131.8107 81.054) (end 133.2425 82.4858) (width 0.2) (layer "B.Cu") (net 15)))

